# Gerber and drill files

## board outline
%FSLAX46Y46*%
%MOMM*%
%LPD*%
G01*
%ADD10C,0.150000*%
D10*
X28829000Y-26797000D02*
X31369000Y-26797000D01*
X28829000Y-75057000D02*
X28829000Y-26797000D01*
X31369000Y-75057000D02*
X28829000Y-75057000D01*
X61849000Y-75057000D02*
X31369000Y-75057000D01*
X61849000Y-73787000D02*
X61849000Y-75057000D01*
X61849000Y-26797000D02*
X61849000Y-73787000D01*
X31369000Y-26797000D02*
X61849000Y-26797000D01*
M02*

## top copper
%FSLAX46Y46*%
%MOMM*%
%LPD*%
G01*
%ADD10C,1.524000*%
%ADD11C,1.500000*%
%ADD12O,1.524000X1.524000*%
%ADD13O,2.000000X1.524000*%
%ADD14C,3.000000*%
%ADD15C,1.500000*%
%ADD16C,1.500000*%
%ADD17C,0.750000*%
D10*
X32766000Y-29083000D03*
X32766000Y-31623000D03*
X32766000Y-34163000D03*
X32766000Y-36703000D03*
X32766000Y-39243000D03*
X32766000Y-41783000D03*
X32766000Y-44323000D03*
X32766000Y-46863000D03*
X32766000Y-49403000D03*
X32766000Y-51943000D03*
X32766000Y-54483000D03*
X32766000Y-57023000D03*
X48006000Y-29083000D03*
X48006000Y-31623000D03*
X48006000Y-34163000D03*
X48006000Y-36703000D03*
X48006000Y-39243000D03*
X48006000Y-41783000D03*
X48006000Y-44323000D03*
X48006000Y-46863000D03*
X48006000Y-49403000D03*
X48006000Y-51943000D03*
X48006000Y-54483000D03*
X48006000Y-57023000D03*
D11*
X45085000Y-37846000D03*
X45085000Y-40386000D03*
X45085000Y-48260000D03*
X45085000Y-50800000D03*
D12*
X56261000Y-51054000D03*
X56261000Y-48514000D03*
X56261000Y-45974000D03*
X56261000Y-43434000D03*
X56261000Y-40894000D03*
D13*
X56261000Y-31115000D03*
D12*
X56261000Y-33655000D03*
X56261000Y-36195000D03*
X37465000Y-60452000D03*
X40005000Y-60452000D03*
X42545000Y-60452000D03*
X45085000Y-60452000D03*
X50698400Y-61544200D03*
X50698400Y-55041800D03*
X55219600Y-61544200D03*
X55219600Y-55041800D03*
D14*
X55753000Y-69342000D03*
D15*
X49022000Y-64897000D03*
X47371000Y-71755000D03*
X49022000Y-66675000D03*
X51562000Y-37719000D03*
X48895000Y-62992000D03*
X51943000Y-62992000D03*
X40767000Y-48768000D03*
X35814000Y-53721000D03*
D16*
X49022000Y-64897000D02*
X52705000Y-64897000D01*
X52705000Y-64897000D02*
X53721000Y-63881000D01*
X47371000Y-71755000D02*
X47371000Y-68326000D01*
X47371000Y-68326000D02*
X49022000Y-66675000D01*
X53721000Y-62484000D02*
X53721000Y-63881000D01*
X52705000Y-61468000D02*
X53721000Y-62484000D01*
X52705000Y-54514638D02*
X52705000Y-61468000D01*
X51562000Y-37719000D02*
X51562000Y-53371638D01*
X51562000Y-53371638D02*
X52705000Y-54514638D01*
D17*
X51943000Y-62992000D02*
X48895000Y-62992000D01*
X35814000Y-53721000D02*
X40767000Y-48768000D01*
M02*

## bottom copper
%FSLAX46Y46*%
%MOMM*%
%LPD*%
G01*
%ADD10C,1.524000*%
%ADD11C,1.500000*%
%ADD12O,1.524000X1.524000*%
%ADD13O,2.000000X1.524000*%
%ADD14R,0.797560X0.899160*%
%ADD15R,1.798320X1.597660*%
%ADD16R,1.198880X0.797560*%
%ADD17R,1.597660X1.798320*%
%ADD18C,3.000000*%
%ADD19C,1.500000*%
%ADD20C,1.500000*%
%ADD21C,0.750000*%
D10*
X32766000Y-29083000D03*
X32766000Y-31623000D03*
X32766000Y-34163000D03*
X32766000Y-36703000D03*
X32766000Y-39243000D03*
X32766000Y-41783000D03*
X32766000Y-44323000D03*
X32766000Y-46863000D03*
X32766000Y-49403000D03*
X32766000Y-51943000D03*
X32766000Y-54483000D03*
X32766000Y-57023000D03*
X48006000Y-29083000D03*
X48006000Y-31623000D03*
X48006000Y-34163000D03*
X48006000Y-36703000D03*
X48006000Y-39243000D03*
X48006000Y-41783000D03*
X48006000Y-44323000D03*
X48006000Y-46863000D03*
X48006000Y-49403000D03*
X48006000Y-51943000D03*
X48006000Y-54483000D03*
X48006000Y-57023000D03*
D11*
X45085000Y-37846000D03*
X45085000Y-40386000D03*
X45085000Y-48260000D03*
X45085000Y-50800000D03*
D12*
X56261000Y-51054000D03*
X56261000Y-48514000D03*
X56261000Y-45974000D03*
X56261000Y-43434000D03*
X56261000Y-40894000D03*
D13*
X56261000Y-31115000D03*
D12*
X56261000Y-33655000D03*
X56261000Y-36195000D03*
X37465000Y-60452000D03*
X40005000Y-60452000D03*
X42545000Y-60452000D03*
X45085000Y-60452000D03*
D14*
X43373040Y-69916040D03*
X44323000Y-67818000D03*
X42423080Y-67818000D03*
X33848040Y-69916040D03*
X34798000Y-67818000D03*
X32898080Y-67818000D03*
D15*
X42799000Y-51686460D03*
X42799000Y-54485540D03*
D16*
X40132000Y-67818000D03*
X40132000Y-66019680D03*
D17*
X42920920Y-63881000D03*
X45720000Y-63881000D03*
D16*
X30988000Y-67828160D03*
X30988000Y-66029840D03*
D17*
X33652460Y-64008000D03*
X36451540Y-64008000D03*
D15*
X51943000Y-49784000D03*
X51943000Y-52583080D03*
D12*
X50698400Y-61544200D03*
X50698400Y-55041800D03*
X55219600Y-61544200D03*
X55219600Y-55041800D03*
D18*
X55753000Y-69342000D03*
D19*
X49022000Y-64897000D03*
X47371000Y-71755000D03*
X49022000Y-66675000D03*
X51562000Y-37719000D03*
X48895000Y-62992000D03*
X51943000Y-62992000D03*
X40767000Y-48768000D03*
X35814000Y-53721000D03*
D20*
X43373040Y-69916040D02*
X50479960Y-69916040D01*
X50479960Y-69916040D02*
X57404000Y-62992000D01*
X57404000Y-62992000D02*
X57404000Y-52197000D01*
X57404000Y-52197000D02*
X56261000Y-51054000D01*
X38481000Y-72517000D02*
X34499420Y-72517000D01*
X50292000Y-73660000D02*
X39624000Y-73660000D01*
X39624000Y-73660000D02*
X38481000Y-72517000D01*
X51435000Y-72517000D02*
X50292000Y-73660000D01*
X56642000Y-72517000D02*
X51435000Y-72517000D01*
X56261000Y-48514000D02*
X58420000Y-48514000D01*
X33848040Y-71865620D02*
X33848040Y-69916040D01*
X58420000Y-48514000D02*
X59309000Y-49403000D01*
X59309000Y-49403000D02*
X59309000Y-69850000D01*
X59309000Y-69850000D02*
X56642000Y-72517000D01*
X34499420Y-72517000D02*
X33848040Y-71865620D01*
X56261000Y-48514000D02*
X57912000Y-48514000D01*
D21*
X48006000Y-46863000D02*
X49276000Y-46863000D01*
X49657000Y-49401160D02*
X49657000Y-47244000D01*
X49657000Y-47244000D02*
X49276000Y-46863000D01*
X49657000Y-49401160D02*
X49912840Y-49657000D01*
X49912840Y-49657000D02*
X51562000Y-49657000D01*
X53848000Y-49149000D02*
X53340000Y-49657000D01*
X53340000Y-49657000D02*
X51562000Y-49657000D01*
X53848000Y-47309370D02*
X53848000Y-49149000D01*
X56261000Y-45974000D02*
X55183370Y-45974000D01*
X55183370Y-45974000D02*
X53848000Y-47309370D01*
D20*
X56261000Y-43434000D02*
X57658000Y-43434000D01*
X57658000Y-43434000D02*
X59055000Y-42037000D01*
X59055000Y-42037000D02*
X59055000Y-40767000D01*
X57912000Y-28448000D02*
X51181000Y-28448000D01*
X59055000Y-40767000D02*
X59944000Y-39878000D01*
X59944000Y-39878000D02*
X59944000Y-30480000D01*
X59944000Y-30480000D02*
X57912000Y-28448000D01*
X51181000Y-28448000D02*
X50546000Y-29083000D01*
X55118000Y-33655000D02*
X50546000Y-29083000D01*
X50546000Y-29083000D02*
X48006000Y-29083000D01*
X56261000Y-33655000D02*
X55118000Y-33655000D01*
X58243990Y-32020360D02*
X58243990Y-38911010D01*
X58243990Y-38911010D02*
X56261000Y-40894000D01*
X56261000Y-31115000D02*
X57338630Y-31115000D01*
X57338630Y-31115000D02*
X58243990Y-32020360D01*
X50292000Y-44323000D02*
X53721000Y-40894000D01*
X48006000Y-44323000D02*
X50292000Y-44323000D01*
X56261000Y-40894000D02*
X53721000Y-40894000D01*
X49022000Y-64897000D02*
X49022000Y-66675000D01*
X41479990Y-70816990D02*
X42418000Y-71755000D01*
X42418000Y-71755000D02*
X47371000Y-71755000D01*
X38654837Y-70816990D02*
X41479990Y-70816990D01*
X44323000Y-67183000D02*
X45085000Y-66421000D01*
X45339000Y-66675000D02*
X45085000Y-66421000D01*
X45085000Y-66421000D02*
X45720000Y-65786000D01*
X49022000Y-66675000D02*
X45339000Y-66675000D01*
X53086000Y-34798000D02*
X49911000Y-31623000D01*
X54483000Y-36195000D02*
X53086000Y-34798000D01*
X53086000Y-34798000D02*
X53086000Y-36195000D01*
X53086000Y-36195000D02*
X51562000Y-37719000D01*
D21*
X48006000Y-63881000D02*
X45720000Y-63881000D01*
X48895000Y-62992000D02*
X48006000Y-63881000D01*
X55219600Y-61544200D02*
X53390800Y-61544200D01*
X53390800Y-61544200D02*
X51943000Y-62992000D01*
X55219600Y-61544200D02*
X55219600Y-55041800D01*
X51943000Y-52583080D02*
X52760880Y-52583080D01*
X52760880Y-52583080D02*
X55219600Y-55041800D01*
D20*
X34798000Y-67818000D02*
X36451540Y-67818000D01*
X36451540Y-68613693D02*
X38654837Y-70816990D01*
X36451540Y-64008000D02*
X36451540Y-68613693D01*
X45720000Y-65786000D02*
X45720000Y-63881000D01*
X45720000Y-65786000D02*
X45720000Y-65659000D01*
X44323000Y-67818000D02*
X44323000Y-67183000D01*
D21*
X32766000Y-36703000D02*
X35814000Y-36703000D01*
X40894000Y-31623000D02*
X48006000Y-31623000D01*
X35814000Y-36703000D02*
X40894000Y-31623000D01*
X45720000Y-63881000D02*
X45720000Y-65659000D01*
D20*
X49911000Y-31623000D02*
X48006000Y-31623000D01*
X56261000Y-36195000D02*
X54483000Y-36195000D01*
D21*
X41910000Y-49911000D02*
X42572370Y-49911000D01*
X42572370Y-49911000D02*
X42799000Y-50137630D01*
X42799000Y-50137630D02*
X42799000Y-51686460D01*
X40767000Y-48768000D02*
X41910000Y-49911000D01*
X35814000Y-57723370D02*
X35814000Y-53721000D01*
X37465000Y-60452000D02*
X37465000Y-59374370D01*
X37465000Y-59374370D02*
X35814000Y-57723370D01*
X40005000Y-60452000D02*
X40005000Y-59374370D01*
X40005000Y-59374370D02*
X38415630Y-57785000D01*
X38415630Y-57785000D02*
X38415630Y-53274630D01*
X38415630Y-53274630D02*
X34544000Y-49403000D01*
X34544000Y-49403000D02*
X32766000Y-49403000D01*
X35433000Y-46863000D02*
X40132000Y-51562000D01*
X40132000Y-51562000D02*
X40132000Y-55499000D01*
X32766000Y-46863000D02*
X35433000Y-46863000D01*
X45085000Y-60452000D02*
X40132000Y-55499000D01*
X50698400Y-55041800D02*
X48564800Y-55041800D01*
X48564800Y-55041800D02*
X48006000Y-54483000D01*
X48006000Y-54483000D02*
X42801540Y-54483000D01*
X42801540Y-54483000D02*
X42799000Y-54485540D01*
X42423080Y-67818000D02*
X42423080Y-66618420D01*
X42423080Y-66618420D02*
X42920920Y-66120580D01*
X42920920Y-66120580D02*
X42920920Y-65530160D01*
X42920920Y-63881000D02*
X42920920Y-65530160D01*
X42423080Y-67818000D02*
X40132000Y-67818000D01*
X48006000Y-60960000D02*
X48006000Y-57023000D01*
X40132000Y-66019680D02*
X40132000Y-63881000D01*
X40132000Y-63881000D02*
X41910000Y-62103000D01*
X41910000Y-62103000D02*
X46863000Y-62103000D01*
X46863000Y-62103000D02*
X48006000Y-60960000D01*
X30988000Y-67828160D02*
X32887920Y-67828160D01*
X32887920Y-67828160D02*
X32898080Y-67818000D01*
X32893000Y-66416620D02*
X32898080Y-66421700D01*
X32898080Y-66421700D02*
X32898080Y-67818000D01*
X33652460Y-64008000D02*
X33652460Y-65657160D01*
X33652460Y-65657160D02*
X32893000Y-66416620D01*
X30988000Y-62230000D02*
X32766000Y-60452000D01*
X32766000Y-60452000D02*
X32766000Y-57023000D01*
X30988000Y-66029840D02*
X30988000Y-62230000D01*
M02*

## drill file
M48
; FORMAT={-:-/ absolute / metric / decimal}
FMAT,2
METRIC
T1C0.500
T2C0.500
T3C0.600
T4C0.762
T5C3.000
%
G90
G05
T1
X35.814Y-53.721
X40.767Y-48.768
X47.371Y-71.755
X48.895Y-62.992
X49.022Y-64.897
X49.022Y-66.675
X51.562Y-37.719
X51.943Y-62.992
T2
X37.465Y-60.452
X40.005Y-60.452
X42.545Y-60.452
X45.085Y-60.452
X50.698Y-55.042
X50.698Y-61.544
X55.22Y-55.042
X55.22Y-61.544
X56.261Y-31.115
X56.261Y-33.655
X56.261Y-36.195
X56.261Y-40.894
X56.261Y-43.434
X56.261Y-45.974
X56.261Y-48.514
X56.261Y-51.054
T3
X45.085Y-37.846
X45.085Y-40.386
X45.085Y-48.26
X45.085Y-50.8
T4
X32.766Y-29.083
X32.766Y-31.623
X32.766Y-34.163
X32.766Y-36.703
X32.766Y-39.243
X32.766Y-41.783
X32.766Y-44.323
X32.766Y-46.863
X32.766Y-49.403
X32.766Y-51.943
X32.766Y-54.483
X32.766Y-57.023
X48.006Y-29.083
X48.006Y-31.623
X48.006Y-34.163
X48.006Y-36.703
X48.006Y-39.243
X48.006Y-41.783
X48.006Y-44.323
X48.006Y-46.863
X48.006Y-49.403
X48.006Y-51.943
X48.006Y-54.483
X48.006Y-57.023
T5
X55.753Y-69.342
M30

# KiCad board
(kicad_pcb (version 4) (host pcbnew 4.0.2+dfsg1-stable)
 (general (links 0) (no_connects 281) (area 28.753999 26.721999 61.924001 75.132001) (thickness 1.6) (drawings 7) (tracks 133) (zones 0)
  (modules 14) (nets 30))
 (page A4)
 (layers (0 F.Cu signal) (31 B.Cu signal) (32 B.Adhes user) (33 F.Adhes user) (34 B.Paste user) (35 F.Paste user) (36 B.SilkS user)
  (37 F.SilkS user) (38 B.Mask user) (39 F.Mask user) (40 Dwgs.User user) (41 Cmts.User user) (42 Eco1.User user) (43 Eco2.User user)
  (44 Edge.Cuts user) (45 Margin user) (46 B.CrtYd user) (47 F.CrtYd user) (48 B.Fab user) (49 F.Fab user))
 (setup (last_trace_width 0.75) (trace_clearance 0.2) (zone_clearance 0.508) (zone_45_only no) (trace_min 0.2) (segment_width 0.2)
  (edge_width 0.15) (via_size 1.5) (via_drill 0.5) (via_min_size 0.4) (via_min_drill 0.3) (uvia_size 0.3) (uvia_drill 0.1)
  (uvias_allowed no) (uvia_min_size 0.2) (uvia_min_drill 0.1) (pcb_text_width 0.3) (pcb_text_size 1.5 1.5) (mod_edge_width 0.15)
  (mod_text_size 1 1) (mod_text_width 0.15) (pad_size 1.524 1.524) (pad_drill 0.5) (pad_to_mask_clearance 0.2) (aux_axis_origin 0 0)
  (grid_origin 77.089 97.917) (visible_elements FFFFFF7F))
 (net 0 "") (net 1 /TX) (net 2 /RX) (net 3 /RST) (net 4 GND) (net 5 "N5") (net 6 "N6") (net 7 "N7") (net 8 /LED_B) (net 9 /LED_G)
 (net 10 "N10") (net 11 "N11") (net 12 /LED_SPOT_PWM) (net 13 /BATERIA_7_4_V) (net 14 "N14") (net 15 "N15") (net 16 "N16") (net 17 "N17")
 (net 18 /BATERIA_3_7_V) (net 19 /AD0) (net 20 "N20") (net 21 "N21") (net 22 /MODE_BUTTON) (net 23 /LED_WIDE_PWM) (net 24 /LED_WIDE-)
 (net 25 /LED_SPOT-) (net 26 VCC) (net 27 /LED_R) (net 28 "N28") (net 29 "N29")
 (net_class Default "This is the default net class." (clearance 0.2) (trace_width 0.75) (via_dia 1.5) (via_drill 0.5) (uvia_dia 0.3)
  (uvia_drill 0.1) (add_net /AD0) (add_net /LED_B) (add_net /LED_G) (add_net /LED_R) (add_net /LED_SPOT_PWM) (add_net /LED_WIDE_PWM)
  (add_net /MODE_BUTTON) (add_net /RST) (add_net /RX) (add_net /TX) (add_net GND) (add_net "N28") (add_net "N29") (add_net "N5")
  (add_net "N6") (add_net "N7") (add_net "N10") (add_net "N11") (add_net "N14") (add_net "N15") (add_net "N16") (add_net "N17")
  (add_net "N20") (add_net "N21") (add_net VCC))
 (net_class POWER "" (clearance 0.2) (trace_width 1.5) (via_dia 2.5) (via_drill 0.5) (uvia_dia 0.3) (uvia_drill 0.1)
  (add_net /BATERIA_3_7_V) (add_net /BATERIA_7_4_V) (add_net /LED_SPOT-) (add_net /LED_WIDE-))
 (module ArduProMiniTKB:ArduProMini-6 (layer F.Cu) (at 30.226 22.733)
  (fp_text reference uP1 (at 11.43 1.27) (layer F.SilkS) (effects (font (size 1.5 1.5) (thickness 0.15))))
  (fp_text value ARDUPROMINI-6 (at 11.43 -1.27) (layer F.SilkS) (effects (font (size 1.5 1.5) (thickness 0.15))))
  (pad 7 thru_hole circle (at 2.54 6.35) (size 1.524 1.524) (drill 0.762) (layers *.Cu *.Mask F.SilkS) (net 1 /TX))
  (pad 8 thru_hole circle (at 2.54 8.89) (size 1.524 1.524) (drill 0.762) (layers *.Cu *.Mask F.SilkS) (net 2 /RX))
  (pad 9 thru_hole circle (at 2.54 11.43) (size 1.524 1.524) (drill 0.762) (layers *.Cu *.Mask F.SilkS) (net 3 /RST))
  (pad 10 thru_hole circle (at 2.54 13.97) (size 1.524 1.524) (drill 0.762) (layers *.Cu *.Mask F.SilkS) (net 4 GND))
  (pad 11 thru_hole circle (at 2.54 16.51) (size 1.524 1.524) (drill 0.762) (layers *.Cu *.Mask F.SilkS) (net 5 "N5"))
  (pad 12 thru_hole circle (at 2.54 19.05) (size 1.524 1.524) (drill 0.762) (layers *.Cu *.Mask F.SilkS) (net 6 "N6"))
  (pad 13 thru_hole circle (at 2.54 21.59) (size 1.524 1.524) (drill 0.762) (layers *.Cu *.Mask F.SilkS) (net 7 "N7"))
  (pad 14 thru_hole circle (at 2.54 24.13) (size 1.524 1.524) (drill 0.762) (layers *.Cu *.Mask F.SilkS) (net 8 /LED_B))
  (pad 15 thru_hole circle (at 2.54 26.67) (size 1.524 1.524) (drill 0.762) (layers *.Cu *.Mask F.SilkS) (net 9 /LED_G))
  (pad 16 thru_hole circle (at 2.54 29.21) (size 1.524 1.524) (drill 0.762) (layers *.Cu *.Mask F.SilkS) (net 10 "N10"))
  (pad 17 thru_hole circle (at 2.54 31.75) (size 1.524 1.524) (drill 0.762) (layers *.Cu *.Mask F.SilkS) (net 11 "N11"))
  (pad 18 thru_hole circle (at 2.54 34.29) (size 1.524 1.524) (drill 0.762) (layers *.Cu *.Mask F.SilkS) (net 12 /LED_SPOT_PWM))
  (pad 19 thru_hole circle (at 17.78 6.35) (size 1.524 1.524) (drill 0.762) (layers *.Cu *.Mask F.SilkS) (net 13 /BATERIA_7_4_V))
  (pad 20 thru_hole circle (at 17.78 8.89) (size 1.524 1.524) (drill 0.762) (layers *.Cu *.Mask F.SilkS) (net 4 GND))
  (pad 21 thru_hole circle (at 17.78 11.43) (size 1.524 1.524) (drill 0.762) (layers *.Cu *.Mask F.SilkS) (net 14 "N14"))
  (pad 22 thru_hole circle (at 17.78 13.97) (size 1.524 1.524) (drill 0.762) (layers *.Cu *.Mask F.SilkS) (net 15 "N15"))
  (pad 23 thru_hole circle (at 17.78 16.51) (size 1.524 1.524) (drill 0.762) (layers *.Cu *.Mask F.SilkS) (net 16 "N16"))
  (pad 24 thru_hole circle (at 17.78 19.05) (size 1.524 1.524) (drill 0.762) (layers *.Cu *.Mask F.SilkS) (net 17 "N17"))
  (pad 25 thru_hole circle (at 17.78 21.59) (size 1.524 1.524) (drill 0.762) (layers *.Cu *.Mask F.SilkS) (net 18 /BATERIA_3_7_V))
  (pad 26 thru_hole circle (at 17.78 24.13) (size 1.524 1.524) (drill 0.762) (layers *.Cu *.Mask F.SilkS) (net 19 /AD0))
  (pad 27 thru_hole circle (at 17.78 26.67) (size 1.524 1.524) (drill 0.762) (layers *.Cu *.Mask F.SilkS) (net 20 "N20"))
  (pad 28 thru_hole circle (at 17.78 29.21) (size 1.524 1.524) (drill 0.762) (layers *.Cu *.Mask F.SilkS) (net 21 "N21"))
  (pad 29 thru_hole circle (at 17.78 31.75) (size 1.524 1.524) (drill 0.762) (layers *.Cu *.Mask F.SilkS) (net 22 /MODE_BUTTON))
  (pad 30 thru_hole circle (at 17.78 34.29) (size 1.524 1.524) (drill 0.762) (layers *.Cu *.Mask F.SilkS) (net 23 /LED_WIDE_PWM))
  (pad 31 thru_hole circle (at 14.859 15.113) (size 1.5 1.5) (drill 0.6) (layers *.Cu *.Mask F.SilkS))
  (pad 32 thru_hole circle (at 14.859 17.653) (size 1.5 1.5) (drill 0.6) (layers *.Cu *.Mask F.SilkS))
  (pad 34 thru_hole circle (at 14.859 25.527) (size 1.5 1.5) (drill 0.6) (layers *.Cu *.Mask F.SilkS))
  (pad 35 thru_hole circle (at 14.859 28.067) (size 1.5 1.5) (drill 0.6) (layers *.Cu *.Mask F.SilkS)))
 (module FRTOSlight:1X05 (layer F.Cu) (at 56.261 51.054 90)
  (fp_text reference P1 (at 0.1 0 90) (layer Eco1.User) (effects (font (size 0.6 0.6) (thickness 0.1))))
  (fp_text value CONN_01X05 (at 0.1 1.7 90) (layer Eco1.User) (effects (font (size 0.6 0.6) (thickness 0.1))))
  (pad 1 thru_hole oval (at 0 0 180) (size 1.524 1.524) (drill 0.5) (layers *.Cu *.Mask) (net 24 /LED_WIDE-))
  (pad 2 thru_hole oval (at 2.54 0 180) (size 1.524 1.524) (drill 0.5) (layers *.Cu *.Mask) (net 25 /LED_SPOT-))
  (pad 3 thru_hole oval (at 5.08 0 180) (size 1.524 1.524) (drill 0.5) (layers *.Cu *.Mask) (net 19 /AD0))
  (pad 4 thru_hole oval (at 7.62 0 180) (size 1.524 1.524) (drill 0.5) (layers *.Cu *.Mask) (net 13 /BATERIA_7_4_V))
  (pad 5 thru_hole oval (at 10.16 0 180) (size 1.524 1.524) (drill 0.5) (layers *.Cu *.Mask) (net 18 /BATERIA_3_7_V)))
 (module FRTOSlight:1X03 (layer F.Cu) (at 56.261 31.115 270)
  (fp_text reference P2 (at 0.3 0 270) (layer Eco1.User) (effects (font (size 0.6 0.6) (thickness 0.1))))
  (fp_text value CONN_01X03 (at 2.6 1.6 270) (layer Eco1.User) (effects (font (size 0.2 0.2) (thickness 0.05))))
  (pad 1 thru_hole oval (at 0 0) (size 2 1.524) (drill 0.5) (layers *.Cu *.Mask) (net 18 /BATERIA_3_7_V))
  (pad 2 thru_hole oval (at 2.54 0) (size 1.524 1.524) (drill 0.5) (layers *.Cu *.Mask) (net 13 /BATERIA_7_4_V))
  (pad 3 thru_hole oval (at 5.08 0) (size 1.524 1.524) (drill 0.5) (layers *.Cu *.Mask) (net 4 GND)))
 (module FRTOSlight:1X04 (layer F.Cu) (at 37.465 60.452)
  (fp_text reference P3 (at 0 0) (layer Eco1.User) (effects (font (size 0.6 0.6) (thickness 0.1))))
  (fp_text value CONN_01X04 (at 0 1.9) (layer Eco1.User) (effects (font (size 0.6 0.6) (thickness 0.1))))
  (pad 1 thru_hole oval (at 0 0 90) (size 1.524 1.524) (drill 0.5) (layers *.Cu *.Mask) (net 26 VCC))
  (pad 2 thru_hole oval (at 2.54 0 90) (size 1.524 1.524) (drill 0.5) (layers *.Cu *.Mask) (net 9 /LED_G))
  (pad 3 thru_hole oval (at 5.08 0 90) (size 1.524 1.524) (drill 0.5) (layers *.Cu *.Mask) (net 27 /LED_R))
  (pad 4 thru_hole oval (at 7.62 0 90) (size 1.524 1.524) (drill 0.5) (layers *.Cu *.Mask) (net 8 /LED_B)))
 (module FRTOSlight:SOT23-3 (layer B.Cu) (at 43.37304 68.81622)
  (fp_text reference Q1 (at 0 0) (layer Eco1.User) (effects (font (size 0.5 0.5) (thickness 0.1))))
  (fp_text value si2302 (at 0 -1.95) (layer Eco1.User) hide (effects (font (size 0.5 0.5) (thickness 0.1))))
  (pad 3 smd rect (at 0 1.09982) (size 0.79756 0.89916) (layers B.Cu B.Paste B.Mask) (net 24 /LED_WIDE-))
  (pad 2 smd rect (at 0.94996 -0.99822) (size 0.79756 0.89916) (layers B.Cu B.Paste B.Mask) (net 4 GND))
  (pad 1 smd rect (at -0.94996 -0.99822) (size 0.79756 0.89916) (layers B.Cu B.Paste B.Mask) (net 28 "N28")))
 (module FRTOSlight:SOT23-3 (layer B.Cu) (at 33.84804 68.81622)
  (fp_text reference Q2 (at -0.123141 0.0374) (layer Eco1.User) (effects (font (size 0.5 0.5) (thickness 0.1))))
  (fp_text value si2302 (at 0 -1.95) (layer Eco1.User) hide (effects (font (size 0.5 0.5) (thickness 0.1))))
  (pad 3 smd rect (at 0 1.09982) (size 0.79756 0.89916) (layers B.Cu B.Paste B.Mask) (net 25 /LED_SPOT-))
  (pad 2 smd rect (at 0.94996 -0.99822) (size 0.79756 0.89916) (layers B.Cu B.Paste B.Mask) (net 4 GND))
  (pad 1 smd rect (at -0.94996 -0.99822) (size 0.79756 0.89916) (layers B.Cu B.Paste B.Mask) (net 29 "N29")))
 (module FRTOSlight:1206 (layer B.Cu) (at 42.799 53.086 270)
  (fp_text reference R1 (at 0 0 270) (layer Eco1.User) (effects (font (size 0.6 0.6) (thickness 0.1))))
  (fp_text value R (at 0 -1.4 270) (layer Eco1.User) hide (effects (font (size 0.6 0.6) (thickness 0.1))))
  (pad 1 smd rect (at -1.39954 0 270) (size 1.59766 1.79832) (layers B.Cu B.Paste B.Mask) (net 26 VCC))
  (pad 2 smd rect (at 1.39954 0 270) (size 1.59766 1.79832) (layers B.Cu B.Paste B.Mask) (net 22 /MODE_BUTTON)))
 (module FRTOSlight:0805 (layer B.Cu) (at 40.132 66.91884 90)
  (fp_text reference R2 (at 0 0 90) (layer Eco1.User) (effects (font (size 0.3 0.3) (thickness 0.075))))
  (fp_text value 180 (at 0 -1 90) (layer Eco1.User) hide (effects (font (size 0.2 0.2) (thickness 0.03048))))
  (pad 1 smd rect (at -0.89916 0 90) (size 0.79756 1.19888) (layers B.Cu B.Paste B.Mask) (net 28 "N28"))
  (pad 2 smd rect (at 0.89916 0 90) (size 0.79756 1.19888) (layers B.Cu B.Paste B.Mask) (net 23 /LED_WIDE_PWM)))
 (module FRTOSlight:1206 (layer B.Cu) (at 44.32046 63.881)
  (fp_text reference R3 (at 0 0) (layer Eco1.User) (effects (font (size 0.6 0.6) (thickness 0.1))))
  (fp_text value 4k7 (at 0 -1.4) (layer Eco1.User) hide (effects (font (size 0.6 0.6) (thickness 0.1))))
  (pad 1 smd rect (at -1.39954 0) (size 1.59766 1.79832) (layers B.Cu B.Paste B.Mask) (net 28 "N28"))
  (pad 2 smd rect (at 1.39954 0) (size 1.59766 1.79832) (layers B.Cu B.Paste B.Mask) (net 4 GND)))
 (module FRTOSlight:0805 (layer B.Cu) (at 30.988 66.929 90)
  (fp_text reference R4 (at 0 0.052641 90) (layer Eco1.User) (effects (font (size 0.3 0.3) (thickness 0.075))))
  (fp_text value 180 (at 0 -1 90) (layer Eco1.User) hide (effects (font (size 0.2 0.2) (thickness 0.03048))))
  (pad 1 smd rect (at -0.89916 0 90) (size 0.79756 1.19888) (layers B.Cu B.Paste B.Mask) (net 29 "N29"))
  (pad 2 smd rect (at 0.89916 0 90) (size 0.79756 1.19888) (layers B.Cu B.Paste B.Mask) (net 12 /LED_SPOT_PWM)))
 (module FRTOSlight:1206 (layer B.Cu) (at 35.052 64.008)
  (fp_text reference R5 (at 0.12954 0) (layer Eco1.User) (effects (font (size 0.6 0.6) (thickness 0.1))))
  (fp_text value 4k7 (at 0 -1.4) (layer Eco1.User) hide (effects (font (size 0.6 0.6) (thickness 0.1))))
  (pad 1 smd rect (at -1.39954 0) (size 1.59766 1.79832) (layers B.Cu B.Paste B.Mask) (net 29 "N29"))
  (pad 2 smd rect (at 1.39954 0) (size 1.59766 1.79832) (layers B.Cu B.Paste B.Mask) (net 4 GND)))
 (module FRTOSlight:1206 (layer B.Cu) (at 51.943 51.18354 270)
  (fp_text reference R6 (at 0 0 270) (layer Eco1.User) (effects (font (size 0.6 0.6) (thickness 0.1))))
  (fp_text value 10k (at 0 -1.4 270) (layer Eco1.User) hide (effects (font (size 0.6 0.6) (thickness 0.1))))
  (pad 1 smd rect (at -1.39954 0 270) (size 1.59766 1.79832) (layers B.Cu B.Paste B.Mask) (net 19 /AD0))
  (pad 2 smd rect (at 1.39954 0 270) (size 1.59766 1.79832) (layers B.Cu B.Paste B.Mask) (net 4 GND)))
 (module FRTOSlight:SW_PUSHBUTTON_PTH (layer F.Cu) (at 52.959 58.293 90)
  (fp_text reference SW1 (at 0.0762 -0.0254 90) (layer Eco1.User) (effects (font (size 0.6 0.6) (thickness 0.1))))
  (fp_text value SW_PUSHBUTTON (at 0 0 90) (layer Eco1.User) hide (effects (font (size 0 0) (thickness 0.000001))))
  (pad 1 thru_hole oval (at -3.2512 -2.2606 90) (size 1.524 1.524) (drill 0.5) (layers *.Cu *.Mask) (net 22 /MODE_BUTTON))
  (pad 1 thru_hole oval (at 3.2512 -2.2606 90) (size 1.524 1.524) (drill 0.5) (layers *.Cu *.Mask) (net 22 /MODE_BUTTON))
  (pad 2 thru_hole oval (at -3.2512 2.2606 90) (size 1.524 1.524) (drill 0.5) (layers *.Cu *.Mask) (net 4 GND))
  (pad 2 thru_hole oval (at 3.2512 2.2606 90) (size 1.524 1.524) (drill 0.5) (layers *.Cu *.Mask) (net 4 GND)))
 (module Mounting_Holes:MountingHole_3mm (layer F.Cu) (at 55.753 69.342)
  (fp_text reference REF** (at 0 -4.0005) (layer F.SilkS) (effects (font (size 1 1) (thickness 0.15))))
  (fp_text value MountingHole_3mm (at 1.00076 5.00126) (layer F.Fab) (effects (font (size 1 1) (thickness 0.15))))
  (pad 1 thru_hole circle (at 0 0) (size 3 3) (drill 3) (layers)))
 (gr_line (start 28.829 26.797) (end 31.369 26.797) (layer Edge.Cuts) (width 0.15))
 (gr_line (start 28.829 75.057) (end 28.829 26.797) (layer Edge.Cuts) (width 0.15))
 (gr_line (start 31.369 75.057) (end 28.829 75.057) (layer Edge.Cuts) (width 0.15))
 (gr_line (start 61.849 75.057) (end 31.369 75.057) (layer Edge.Cuts) (width 0.15))
 (gr_line (start 61.849 73.787) (end 61.849 75.057) (layer Edge.Cuts) (width 0.15))
 (gr_line (start 61.849 26.797) (end 61.849 73.787) (layer Edge.Cuts) (width 0.15))
 (gr_line (start 31.369 26.797) (end 61.849 26.797) (layer Edge.Cuts) (width 0.15))
 (segment (start 43.37304 69.91604) (end 50.47996 69.91604) (width 1.5) (layer B.Cu) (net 24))
 (segment (start 50.47996 69.91604) (end 57.404 62.992) (width 1.5) (layer B.Cu) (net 24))
 (segment (start 57.404 62.992) (end 57.404 52.197) (width 1.5) (layer B.Cu) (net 24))
 (segment (start 57.404 52.197) (end 56.261 51.054) (width 1.5) (layer B.Cu) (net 24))
 (segment (start 38.481 72.517) (end 34.49942 72.517) (width 1.5) (layer B.Cu) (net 25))
 (segment (start 50.292 73.66) (end 39.624 73.66) (width 1.5) (layer B.Cu) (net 25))
 (segment (start 39.624 73.66) (end 38.481 72.517) (width 1.5) (layer B.Cu) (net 25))
 (segment (start 51.435 72.517) (end 50.292 73.66) (width 1.5) (layer B.Cu) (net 25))
 (segment (start 56.642 72.517) (end 51.435 72.517) (width 1.5) (layer B.Cu) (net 25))
 (segment (start 56.261 48.514) (end 58.42 48.514) (width 1.5) (layer B.Cu) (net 25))
 (segment (start 33.84804 71.86562) (end 33.84804 69.91604) (width 1.5) (layer B.Cu) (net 25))
 (segment (start 58.42 48.514) (end 59.309 49.403) (width 1.5) (layer B.Cu) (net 25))
 (segment (start 59.309 49.403) (end 59.309 69.85) (width 1.5) (layer B.Cu) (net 25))
 (segment (start 59.309 69.85) (end 56.642 72.517) (width 1.5) (layer B.Cu) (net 25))
 (segment (start 34.49942 72.517) (end 33.84804 71.86562) (width 1.5) (layer B.Cu) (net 25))
 (segment (start 56.261 48.514) (end 57.912 48.514) (width 1.5) (layer B.Cu) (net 25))
 (segment (start 48.006 46.863) (end 49.276 46.863) (width 0.75) (layer B.Cu) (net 19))
 (segment (start 49.657 49.40116) (end 49.657 47.244) (width 0.75) (layer B.Cu) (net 19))
 (segment (start 49.657 47.244) (end 49.276 46.863) (width 0.75) (layer B.Cu) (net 19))
 (segment (start 49.657 49.40116) (end 49.91284 49.657) (width 0.75) (layer B.Cu) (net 19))
 (segment (start 49.91284 49.657) (end 51.562 49.657) (width 0.75) (layer B.Cu) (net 19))
 (segment (start 53.848 49.149) (end 53.34 49.657) (width 0.75) (layer B.Cu) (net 19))
 (segment (start 53.34 49.657) (end 51.562 49.657) (width 0.75) (layer B.Cu) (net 19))
 (segment (start 53.848 47.30937) (end 53.848 49.149) (width 0.75) (layer B.Cu) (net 19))
 (segment (start 56.261 45.974) (end 55.18337 45.974) (width 0.75) (layer B.Cu) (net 19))
 (segment (start 55.18337 45.974) (end 53.848 47.30937) (width 0.75) (layer B.Cu) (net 19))
 (segment (start 56.261 43.434) (end 57.658 43.434) (width 1.5) (layer B.Cu) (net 13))
 (segment (start 57.658 43.434) (end 59.055 42.037) (width 1.5) (layer B.Cu) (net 13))
 (segment (start 59.055 42.037) (end 59.055 40.767) (width 1.5) (layer B.Cu) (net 13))
 (segment (start 57.912 28.448) (end 51.181 28.448) (width 1.5) (layer B.Cu) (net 13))
 (segment (start 59.055 40.767) (end 59.944 39.878) (width 1.5) (layer B.Cu) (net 13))
 (segment (start 59.944 39.878) (end 59.944 30.48) (width 1.5) (layer B.Cu) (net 13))
 (segment (start 59.944 30.48) (end 57.912 28.448) (width 1.5) (layer B.Cu) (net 13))
 (segment (start 51.181 28.448) (end 50.546 29.083) (width 1.5) (layer B.Cu) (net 13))
 (segment (start 55.118 33.655) (end 50.546 29.083) (width 1.5) (layer B.Cu) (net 13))
 (segment (start 50.546 29.083) (end 48.006 29.083) (width 1.5) (layer B.Cu) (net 13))
 (segment (start 56.261 33.655) (end 55.118 33.655) (width 1.5) (layer B.Cu) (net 13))
 (segment (start 58.24399 32.02036) (end 58.24399 38.91101) (width 1.5) (layer B.Cu) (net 18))
 (segment (start 58.24399 38.91101) (end 56.261 40.894) (width 1.5) (layer B.Cu) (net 18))
 (segment (start 56.261 31.115) (end 57.33863 31.115) (width 1.5) (layer B.Cu) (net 18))
 (segment (start 57.33863 31.115) (end 58.24399 32.02036) (width 1.5) (layer B.Cu) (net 18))
 (segment (start 50.292 44.323) (end 53.721 40.894) (width 1.5) (layer B.Cu) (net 18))
 (segment (start 48.006 44.323) (end 50.292 44.323) (width 1.5) (layer B.Cu) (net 18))
 (segment (start 56.261 40.894) (end 53.721 40.894) (width 1.5) (layer B.Cu) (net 18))
 (segment (start 49.022 64.897) (end 52.705 64.897) (width 1.5) (layer F.Cu) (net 4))
 (segment (start 52.705 64.897) (end 53.721 63.881) (width 1.5) (layer F.Cu) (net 4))
 (segment (start 47.371 71.755) (end 47.371 68.326) (width 1.5) (layer F.Cu) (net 4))
 (segment (start 47.371 68.326) (end 49.022 66.675) (width 1.5) (layer F.Cu) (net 4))
 (segment (start 49.022 64.897) (end 49.022 66.675) (width 1.5) (layer B.Cu) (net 4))
 (via (at 49.022 64.897) (size 1.5) (drill 0.5) (layers F.Cu B.Cu) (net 4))
 (segment (start 41.47999 70.81699) (end 42.418 71.755) (width 1.5) (layer B.Cu) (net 4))
 (segment (start 42.418 71.755) (end 47.371 71.755) (width 1.5) (layer B.Cu) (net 4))
 (via (at 47.371 71.755) (size 1.5) (drill 0.5) (layers F.Cu B.Cu) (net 4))
 (segment (start 38.654837 70.81699) (end 41.47999 70.81699) (width 1.5) (layer B.Cu) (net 4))
 (segment (start 44.323 67.183) (end 45.085 66.421) (width 1.5) (layer B.Cu) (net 4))
 (segment (start 45.339 66.675) (end 45.085 66.421) (width 1.5) (layer B.Cu) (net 4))
 (segment (start 45.085 66.421) (end 45.72 65.786) (width 1.5) (layer B.Cu) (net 4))
 (segment (start 49.022 66.675) (end 45.339 66.675) (width 1.5) (layer B.Cu) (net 4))
 (via (at 49.022 66.675) (size 1.5) (drill 0.5) (layers F.Cu B.Cu) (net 4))
 (segment (start 53.721 62.484) (end 53.721 63.881) (width 1.5) (layer F.Cu) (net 4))
 (segment (start 52.705 61.468) (end 53.721 62.484) (width 1.5) (layer F.Cu) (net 4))
 (segment (start 52.705 54.514638) (end 52.705 61.468) (width 1.5) (layer F.Cu) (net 4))
 (segment (start 51.562 37.719) (end 51.562 53.371638) (width 1.5) (layer F.Cu) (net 4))
 (segment (start 51.562 53.371638) (end 52.705 54.514638) (width 1.5) (layer F.Cu) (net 4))
 (segment (start 53.086 34.798) (end 49.911 31.623) (width 1.5) (layer B.Cu) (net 4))
 (segment (start 54.483 36.195) (end 53.086 34.798) (width 1.5) (layer B.Cu) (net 4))
 (segment (start 53.086 34.798) (end 53.086 36.195) (width 1.5) (layer B.Cu) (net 4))
 (segment (start 53.086 36.195) (end 51.562 37.719) (width 1.5) (layer B.Cu) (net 4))
 (via (at 51.562 37.719) (size 1.5) (drill 0.5) (layers F.Cu B.Cu) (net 4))
 (segment (start 48.006 63.881) (end 45.72 63.881) (width 0.75) (layer B.Cu) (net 4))
 (segment (start 48.895 62.992) (end 48.006 63.881) (width 0.75) (layer B.Cu) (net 4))
 (segment (start 55.2196 61.5442) (end 53.3908 61.5442) (width 0.75) (layer B.Cu) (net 4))
 (segment (start 53.3908 61.5442) (end 51.943 62.992) (width 0.75) (layer B.Cu) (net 4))
 (segment (start 55.2196 61.5442) (end 55.2196 55.0418) (width 0.75) (layer B.Cu) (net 4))
 (segment (start 51.943 52.58308) (end 52.76088 52.58308) (width 0.75) (layer B.Cu) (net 4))
 (segment (start 52.76088 52.58308) (end 55.2196 55.0418) (width 0.75) (layer B.Cu) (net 4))
 (segment (start 34.798 67.818) (end 36.45154 67.818) (width 1.5) (layer B.Cu) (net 4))
 (segment (start 36.45154 68.613693) (end 38.654837 70.81699) (width 1.5) (layer B.Cu) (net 4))
 (segment (start 36.45154 64.008) (end 36.45154 68.613693) (width 1.5) (layer B.Cu) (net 4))
 (segment (start 45.72 65.786) (end 45.72 63.881) (width 1.5) (layer B.Cu) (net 4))
 (segment (start 45.72 65.786) (end 45.72 65.659) (width 1.5) (layer B.Cu) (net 4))
 (segment (start 44.323 67.818) (end 44.323 67.183) (width 1.5) (layer B.Cu) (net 4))
 (segment (start 32.766 36.703) (end 35.814 36.703) (width 0.75) (layer B.Cu) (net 4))
 (segment (start 40.894 31.623) (end 48.006 31.623) (width 0.75) (layer B.Cu) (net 4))
 (segment (start 35.814 36.703) (end 40.894 31.623) (width 0.75) (layer B.Cu) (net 4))
 (segment (start 51.943 62.992) (end 48.895 62.992) (width 0.75) (layer F.Cu) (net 4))
 (via (at 48.895 62.992) (size 1.5) (drill 0.5) (layers F.Cu B.Cu) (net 4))
 (via (at 51.943 62.992) (size 1.5) (drill 0.5) (layers F.Cu B.Cu) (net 4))
 (segment (start 45.72 63.881) (end 45.72 65.659) (width 0.75) (layer B.Cu) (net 4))
 (segment (start 49.911 31.623) (end 48.006 31.623) (width 1.5) (layer B.Cu) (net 4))
 (segment (start 56.261 36.195) (end 54.483 36.195) (width 1.5) (layer B.Cu) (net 4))
 (segment (start 41.91 49.911) (end 42.57237 49.911) (width 0.75) (layer B.Cu) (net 26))
 (segment (start 42.57237 49.911) (end 42.799 50.13763) (width 0.75) (layer B.Cu) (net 26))
 (segment (start 42.799 50.13763) (end 42.799 51.68646) (width 0.75) (layer B.Cu) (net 26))
 (segment (start 40.767 48.768) (end 41.91 49.911) (width 0.75) (layer B.Cu) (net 26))
 (segment (start 35.814 53.721) (end 40.767 48.768) (width 0.75) (layer F.Cu) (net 26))
 (via (at 40.767 48.768) (size 1.5) (drill 0.5) (layers F.Cu B.Cu) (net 26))
 (segment (start 35.814 57.72337) (end 35.814 53.721) (width 0.75) (layer B.Cu) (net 26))
 (via (at 35.814 53.721) (size 1.5) (drill 0.5) (layers F.Cu B.Cu) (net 26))
 (segment (start 37.465 60.452) (end 37.465 59.37437) (width 0.75) (layer B.Cu) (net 26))
 (segment (start 37.465 59.37437) (end 35.814 57.72337) (width 0.75) (layer B.Cu) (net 26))
 (segment (start 40.005 60.452) (end 40.005 59.37437) (width 0.75) (layer B.Cu) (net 9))
 (segment (start 40.005 59.37437) (end 38.41563 57.785) (width 0.75) (layer B.Cu) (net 9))
 (segment (start 38.41563 57.785) (end 38.41563 53.27463) (width 0.75) (layer B.Cu) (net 9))
 (segment (start 38.41563 53.27463) (end 34.544 49.403) (width 0.75) (layer B.Cu) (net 9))
 (segment (start 34.544 49.403) (end 32.766 49.403) (width 0.75) (layer B.Cu) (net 9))
 (segment (start 35.433 46.863) (end 40.132 51.562) (width 0.75) (layer B.Cu) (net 8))
 (segment (start 40.132 51.562) (end 40.132 55.499) (width 0.75) (layer B.Cu) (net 8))
 (segment (start 32.766 46.863) (end 35.433 46.863) (width 0.75) (layer B.Cu) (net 8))
 (segment (start 45.085 60.452) (end 40.132 55.499) (width 0.75) (layer B.Cu) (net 8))
 (segment (start 50.6984 55.0418) (end 48.5648 55.0418) (width 0.75) (layer B.Cu) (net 22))
 (segment (start 48.5648 55.0418) (end 48.006 54.483) (width 0.75) (layer B.Cu) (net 22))
 (segment (start 48.006 54.483) (end 42.80154 54.483) (width 0.75) (layer B.Cu) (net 22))
 (segment (start 42.80154 54.483) (end 42.799 54.48554) (width 0.75) (layer B.Cu) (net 22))
 (segment (start 42.42308 67.818) (end 42.42308 66.61842) (width 0.75) (layer B.Cu) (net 28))
 (segment (start 42.42308 66.61842) (end 42.92092 66.12058) (width 0.75) (layer B.Cu) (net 28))
 (segment (start 42.92092 66.12058) (end 42.92092 65.53016) (width 0.75) (layer B.Cu) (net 28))
 (segment (start 42.92092 63.881) (end 42.92092 65.53016) (width 0.75) (layer B.Cu) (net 28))
 (segment (start 42.42308 67.818) (end 40.132 67.818) (width 0.75) (layer B.Cu) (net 28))
 (segment (start 48.006 60.96) (end 48.006 57.023) (width 0.75) (layer B.Cu) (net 23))
 (segment (start 40.132 66.01968) (end 40.132 63.881) (width 0.75) (layer B.Cu) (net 23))
 (segment (start 40.132 63.881) (end 41.91 62.103) (width 0.75) (layer B.Cu) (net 23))
 (segment (start 41.91 62.103) (end 46.863 62.103) (width 0.75) (layer B.Cu) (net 23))
 (segment (start 46.863 62.103) (end 48.006 60.96) (width 0.75) (layer B.Cu) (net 23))
 (segment (start 30.988 67.82816) (end 32.88792 67.82816) (width 0.75) (layer B.Cu) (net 29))
 (segment (start 32.88792 67.82816) (end 32.89808 67.818) (width 0.75) (layer B.Cu) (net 29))
 (segment (start 32.893 66.41662) (end 32.89808 66.4217) (width 0.75) (layer B.Cu) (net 29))
 (segment (start 32.89808 66.4217) (end 32.89808 67.818) (width 0.75) (layer B.Cu) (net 29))
 (segment (start 33.65246 64.008) (end 33.65246 65.65716) (width 0.75) (layer B.Cu) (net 29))
 (segment (start 33.65246 65.65716) (end 32.893 66.41662) (width 0.75) (layer B.Cu) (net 29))
 (segment (start 30.988 62.23) (end 32.766 60.452) (width 0.75) (layer B.Cu) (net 12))
 (segment (start 32.766 60.452) (end 32.766 57.023) (width 0.75) (layer B.Cu) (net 12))
 (segment (start 30.988 66.02984) (end 30.988 62.23) (width 0.75) (layer B.Cu) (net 12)))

